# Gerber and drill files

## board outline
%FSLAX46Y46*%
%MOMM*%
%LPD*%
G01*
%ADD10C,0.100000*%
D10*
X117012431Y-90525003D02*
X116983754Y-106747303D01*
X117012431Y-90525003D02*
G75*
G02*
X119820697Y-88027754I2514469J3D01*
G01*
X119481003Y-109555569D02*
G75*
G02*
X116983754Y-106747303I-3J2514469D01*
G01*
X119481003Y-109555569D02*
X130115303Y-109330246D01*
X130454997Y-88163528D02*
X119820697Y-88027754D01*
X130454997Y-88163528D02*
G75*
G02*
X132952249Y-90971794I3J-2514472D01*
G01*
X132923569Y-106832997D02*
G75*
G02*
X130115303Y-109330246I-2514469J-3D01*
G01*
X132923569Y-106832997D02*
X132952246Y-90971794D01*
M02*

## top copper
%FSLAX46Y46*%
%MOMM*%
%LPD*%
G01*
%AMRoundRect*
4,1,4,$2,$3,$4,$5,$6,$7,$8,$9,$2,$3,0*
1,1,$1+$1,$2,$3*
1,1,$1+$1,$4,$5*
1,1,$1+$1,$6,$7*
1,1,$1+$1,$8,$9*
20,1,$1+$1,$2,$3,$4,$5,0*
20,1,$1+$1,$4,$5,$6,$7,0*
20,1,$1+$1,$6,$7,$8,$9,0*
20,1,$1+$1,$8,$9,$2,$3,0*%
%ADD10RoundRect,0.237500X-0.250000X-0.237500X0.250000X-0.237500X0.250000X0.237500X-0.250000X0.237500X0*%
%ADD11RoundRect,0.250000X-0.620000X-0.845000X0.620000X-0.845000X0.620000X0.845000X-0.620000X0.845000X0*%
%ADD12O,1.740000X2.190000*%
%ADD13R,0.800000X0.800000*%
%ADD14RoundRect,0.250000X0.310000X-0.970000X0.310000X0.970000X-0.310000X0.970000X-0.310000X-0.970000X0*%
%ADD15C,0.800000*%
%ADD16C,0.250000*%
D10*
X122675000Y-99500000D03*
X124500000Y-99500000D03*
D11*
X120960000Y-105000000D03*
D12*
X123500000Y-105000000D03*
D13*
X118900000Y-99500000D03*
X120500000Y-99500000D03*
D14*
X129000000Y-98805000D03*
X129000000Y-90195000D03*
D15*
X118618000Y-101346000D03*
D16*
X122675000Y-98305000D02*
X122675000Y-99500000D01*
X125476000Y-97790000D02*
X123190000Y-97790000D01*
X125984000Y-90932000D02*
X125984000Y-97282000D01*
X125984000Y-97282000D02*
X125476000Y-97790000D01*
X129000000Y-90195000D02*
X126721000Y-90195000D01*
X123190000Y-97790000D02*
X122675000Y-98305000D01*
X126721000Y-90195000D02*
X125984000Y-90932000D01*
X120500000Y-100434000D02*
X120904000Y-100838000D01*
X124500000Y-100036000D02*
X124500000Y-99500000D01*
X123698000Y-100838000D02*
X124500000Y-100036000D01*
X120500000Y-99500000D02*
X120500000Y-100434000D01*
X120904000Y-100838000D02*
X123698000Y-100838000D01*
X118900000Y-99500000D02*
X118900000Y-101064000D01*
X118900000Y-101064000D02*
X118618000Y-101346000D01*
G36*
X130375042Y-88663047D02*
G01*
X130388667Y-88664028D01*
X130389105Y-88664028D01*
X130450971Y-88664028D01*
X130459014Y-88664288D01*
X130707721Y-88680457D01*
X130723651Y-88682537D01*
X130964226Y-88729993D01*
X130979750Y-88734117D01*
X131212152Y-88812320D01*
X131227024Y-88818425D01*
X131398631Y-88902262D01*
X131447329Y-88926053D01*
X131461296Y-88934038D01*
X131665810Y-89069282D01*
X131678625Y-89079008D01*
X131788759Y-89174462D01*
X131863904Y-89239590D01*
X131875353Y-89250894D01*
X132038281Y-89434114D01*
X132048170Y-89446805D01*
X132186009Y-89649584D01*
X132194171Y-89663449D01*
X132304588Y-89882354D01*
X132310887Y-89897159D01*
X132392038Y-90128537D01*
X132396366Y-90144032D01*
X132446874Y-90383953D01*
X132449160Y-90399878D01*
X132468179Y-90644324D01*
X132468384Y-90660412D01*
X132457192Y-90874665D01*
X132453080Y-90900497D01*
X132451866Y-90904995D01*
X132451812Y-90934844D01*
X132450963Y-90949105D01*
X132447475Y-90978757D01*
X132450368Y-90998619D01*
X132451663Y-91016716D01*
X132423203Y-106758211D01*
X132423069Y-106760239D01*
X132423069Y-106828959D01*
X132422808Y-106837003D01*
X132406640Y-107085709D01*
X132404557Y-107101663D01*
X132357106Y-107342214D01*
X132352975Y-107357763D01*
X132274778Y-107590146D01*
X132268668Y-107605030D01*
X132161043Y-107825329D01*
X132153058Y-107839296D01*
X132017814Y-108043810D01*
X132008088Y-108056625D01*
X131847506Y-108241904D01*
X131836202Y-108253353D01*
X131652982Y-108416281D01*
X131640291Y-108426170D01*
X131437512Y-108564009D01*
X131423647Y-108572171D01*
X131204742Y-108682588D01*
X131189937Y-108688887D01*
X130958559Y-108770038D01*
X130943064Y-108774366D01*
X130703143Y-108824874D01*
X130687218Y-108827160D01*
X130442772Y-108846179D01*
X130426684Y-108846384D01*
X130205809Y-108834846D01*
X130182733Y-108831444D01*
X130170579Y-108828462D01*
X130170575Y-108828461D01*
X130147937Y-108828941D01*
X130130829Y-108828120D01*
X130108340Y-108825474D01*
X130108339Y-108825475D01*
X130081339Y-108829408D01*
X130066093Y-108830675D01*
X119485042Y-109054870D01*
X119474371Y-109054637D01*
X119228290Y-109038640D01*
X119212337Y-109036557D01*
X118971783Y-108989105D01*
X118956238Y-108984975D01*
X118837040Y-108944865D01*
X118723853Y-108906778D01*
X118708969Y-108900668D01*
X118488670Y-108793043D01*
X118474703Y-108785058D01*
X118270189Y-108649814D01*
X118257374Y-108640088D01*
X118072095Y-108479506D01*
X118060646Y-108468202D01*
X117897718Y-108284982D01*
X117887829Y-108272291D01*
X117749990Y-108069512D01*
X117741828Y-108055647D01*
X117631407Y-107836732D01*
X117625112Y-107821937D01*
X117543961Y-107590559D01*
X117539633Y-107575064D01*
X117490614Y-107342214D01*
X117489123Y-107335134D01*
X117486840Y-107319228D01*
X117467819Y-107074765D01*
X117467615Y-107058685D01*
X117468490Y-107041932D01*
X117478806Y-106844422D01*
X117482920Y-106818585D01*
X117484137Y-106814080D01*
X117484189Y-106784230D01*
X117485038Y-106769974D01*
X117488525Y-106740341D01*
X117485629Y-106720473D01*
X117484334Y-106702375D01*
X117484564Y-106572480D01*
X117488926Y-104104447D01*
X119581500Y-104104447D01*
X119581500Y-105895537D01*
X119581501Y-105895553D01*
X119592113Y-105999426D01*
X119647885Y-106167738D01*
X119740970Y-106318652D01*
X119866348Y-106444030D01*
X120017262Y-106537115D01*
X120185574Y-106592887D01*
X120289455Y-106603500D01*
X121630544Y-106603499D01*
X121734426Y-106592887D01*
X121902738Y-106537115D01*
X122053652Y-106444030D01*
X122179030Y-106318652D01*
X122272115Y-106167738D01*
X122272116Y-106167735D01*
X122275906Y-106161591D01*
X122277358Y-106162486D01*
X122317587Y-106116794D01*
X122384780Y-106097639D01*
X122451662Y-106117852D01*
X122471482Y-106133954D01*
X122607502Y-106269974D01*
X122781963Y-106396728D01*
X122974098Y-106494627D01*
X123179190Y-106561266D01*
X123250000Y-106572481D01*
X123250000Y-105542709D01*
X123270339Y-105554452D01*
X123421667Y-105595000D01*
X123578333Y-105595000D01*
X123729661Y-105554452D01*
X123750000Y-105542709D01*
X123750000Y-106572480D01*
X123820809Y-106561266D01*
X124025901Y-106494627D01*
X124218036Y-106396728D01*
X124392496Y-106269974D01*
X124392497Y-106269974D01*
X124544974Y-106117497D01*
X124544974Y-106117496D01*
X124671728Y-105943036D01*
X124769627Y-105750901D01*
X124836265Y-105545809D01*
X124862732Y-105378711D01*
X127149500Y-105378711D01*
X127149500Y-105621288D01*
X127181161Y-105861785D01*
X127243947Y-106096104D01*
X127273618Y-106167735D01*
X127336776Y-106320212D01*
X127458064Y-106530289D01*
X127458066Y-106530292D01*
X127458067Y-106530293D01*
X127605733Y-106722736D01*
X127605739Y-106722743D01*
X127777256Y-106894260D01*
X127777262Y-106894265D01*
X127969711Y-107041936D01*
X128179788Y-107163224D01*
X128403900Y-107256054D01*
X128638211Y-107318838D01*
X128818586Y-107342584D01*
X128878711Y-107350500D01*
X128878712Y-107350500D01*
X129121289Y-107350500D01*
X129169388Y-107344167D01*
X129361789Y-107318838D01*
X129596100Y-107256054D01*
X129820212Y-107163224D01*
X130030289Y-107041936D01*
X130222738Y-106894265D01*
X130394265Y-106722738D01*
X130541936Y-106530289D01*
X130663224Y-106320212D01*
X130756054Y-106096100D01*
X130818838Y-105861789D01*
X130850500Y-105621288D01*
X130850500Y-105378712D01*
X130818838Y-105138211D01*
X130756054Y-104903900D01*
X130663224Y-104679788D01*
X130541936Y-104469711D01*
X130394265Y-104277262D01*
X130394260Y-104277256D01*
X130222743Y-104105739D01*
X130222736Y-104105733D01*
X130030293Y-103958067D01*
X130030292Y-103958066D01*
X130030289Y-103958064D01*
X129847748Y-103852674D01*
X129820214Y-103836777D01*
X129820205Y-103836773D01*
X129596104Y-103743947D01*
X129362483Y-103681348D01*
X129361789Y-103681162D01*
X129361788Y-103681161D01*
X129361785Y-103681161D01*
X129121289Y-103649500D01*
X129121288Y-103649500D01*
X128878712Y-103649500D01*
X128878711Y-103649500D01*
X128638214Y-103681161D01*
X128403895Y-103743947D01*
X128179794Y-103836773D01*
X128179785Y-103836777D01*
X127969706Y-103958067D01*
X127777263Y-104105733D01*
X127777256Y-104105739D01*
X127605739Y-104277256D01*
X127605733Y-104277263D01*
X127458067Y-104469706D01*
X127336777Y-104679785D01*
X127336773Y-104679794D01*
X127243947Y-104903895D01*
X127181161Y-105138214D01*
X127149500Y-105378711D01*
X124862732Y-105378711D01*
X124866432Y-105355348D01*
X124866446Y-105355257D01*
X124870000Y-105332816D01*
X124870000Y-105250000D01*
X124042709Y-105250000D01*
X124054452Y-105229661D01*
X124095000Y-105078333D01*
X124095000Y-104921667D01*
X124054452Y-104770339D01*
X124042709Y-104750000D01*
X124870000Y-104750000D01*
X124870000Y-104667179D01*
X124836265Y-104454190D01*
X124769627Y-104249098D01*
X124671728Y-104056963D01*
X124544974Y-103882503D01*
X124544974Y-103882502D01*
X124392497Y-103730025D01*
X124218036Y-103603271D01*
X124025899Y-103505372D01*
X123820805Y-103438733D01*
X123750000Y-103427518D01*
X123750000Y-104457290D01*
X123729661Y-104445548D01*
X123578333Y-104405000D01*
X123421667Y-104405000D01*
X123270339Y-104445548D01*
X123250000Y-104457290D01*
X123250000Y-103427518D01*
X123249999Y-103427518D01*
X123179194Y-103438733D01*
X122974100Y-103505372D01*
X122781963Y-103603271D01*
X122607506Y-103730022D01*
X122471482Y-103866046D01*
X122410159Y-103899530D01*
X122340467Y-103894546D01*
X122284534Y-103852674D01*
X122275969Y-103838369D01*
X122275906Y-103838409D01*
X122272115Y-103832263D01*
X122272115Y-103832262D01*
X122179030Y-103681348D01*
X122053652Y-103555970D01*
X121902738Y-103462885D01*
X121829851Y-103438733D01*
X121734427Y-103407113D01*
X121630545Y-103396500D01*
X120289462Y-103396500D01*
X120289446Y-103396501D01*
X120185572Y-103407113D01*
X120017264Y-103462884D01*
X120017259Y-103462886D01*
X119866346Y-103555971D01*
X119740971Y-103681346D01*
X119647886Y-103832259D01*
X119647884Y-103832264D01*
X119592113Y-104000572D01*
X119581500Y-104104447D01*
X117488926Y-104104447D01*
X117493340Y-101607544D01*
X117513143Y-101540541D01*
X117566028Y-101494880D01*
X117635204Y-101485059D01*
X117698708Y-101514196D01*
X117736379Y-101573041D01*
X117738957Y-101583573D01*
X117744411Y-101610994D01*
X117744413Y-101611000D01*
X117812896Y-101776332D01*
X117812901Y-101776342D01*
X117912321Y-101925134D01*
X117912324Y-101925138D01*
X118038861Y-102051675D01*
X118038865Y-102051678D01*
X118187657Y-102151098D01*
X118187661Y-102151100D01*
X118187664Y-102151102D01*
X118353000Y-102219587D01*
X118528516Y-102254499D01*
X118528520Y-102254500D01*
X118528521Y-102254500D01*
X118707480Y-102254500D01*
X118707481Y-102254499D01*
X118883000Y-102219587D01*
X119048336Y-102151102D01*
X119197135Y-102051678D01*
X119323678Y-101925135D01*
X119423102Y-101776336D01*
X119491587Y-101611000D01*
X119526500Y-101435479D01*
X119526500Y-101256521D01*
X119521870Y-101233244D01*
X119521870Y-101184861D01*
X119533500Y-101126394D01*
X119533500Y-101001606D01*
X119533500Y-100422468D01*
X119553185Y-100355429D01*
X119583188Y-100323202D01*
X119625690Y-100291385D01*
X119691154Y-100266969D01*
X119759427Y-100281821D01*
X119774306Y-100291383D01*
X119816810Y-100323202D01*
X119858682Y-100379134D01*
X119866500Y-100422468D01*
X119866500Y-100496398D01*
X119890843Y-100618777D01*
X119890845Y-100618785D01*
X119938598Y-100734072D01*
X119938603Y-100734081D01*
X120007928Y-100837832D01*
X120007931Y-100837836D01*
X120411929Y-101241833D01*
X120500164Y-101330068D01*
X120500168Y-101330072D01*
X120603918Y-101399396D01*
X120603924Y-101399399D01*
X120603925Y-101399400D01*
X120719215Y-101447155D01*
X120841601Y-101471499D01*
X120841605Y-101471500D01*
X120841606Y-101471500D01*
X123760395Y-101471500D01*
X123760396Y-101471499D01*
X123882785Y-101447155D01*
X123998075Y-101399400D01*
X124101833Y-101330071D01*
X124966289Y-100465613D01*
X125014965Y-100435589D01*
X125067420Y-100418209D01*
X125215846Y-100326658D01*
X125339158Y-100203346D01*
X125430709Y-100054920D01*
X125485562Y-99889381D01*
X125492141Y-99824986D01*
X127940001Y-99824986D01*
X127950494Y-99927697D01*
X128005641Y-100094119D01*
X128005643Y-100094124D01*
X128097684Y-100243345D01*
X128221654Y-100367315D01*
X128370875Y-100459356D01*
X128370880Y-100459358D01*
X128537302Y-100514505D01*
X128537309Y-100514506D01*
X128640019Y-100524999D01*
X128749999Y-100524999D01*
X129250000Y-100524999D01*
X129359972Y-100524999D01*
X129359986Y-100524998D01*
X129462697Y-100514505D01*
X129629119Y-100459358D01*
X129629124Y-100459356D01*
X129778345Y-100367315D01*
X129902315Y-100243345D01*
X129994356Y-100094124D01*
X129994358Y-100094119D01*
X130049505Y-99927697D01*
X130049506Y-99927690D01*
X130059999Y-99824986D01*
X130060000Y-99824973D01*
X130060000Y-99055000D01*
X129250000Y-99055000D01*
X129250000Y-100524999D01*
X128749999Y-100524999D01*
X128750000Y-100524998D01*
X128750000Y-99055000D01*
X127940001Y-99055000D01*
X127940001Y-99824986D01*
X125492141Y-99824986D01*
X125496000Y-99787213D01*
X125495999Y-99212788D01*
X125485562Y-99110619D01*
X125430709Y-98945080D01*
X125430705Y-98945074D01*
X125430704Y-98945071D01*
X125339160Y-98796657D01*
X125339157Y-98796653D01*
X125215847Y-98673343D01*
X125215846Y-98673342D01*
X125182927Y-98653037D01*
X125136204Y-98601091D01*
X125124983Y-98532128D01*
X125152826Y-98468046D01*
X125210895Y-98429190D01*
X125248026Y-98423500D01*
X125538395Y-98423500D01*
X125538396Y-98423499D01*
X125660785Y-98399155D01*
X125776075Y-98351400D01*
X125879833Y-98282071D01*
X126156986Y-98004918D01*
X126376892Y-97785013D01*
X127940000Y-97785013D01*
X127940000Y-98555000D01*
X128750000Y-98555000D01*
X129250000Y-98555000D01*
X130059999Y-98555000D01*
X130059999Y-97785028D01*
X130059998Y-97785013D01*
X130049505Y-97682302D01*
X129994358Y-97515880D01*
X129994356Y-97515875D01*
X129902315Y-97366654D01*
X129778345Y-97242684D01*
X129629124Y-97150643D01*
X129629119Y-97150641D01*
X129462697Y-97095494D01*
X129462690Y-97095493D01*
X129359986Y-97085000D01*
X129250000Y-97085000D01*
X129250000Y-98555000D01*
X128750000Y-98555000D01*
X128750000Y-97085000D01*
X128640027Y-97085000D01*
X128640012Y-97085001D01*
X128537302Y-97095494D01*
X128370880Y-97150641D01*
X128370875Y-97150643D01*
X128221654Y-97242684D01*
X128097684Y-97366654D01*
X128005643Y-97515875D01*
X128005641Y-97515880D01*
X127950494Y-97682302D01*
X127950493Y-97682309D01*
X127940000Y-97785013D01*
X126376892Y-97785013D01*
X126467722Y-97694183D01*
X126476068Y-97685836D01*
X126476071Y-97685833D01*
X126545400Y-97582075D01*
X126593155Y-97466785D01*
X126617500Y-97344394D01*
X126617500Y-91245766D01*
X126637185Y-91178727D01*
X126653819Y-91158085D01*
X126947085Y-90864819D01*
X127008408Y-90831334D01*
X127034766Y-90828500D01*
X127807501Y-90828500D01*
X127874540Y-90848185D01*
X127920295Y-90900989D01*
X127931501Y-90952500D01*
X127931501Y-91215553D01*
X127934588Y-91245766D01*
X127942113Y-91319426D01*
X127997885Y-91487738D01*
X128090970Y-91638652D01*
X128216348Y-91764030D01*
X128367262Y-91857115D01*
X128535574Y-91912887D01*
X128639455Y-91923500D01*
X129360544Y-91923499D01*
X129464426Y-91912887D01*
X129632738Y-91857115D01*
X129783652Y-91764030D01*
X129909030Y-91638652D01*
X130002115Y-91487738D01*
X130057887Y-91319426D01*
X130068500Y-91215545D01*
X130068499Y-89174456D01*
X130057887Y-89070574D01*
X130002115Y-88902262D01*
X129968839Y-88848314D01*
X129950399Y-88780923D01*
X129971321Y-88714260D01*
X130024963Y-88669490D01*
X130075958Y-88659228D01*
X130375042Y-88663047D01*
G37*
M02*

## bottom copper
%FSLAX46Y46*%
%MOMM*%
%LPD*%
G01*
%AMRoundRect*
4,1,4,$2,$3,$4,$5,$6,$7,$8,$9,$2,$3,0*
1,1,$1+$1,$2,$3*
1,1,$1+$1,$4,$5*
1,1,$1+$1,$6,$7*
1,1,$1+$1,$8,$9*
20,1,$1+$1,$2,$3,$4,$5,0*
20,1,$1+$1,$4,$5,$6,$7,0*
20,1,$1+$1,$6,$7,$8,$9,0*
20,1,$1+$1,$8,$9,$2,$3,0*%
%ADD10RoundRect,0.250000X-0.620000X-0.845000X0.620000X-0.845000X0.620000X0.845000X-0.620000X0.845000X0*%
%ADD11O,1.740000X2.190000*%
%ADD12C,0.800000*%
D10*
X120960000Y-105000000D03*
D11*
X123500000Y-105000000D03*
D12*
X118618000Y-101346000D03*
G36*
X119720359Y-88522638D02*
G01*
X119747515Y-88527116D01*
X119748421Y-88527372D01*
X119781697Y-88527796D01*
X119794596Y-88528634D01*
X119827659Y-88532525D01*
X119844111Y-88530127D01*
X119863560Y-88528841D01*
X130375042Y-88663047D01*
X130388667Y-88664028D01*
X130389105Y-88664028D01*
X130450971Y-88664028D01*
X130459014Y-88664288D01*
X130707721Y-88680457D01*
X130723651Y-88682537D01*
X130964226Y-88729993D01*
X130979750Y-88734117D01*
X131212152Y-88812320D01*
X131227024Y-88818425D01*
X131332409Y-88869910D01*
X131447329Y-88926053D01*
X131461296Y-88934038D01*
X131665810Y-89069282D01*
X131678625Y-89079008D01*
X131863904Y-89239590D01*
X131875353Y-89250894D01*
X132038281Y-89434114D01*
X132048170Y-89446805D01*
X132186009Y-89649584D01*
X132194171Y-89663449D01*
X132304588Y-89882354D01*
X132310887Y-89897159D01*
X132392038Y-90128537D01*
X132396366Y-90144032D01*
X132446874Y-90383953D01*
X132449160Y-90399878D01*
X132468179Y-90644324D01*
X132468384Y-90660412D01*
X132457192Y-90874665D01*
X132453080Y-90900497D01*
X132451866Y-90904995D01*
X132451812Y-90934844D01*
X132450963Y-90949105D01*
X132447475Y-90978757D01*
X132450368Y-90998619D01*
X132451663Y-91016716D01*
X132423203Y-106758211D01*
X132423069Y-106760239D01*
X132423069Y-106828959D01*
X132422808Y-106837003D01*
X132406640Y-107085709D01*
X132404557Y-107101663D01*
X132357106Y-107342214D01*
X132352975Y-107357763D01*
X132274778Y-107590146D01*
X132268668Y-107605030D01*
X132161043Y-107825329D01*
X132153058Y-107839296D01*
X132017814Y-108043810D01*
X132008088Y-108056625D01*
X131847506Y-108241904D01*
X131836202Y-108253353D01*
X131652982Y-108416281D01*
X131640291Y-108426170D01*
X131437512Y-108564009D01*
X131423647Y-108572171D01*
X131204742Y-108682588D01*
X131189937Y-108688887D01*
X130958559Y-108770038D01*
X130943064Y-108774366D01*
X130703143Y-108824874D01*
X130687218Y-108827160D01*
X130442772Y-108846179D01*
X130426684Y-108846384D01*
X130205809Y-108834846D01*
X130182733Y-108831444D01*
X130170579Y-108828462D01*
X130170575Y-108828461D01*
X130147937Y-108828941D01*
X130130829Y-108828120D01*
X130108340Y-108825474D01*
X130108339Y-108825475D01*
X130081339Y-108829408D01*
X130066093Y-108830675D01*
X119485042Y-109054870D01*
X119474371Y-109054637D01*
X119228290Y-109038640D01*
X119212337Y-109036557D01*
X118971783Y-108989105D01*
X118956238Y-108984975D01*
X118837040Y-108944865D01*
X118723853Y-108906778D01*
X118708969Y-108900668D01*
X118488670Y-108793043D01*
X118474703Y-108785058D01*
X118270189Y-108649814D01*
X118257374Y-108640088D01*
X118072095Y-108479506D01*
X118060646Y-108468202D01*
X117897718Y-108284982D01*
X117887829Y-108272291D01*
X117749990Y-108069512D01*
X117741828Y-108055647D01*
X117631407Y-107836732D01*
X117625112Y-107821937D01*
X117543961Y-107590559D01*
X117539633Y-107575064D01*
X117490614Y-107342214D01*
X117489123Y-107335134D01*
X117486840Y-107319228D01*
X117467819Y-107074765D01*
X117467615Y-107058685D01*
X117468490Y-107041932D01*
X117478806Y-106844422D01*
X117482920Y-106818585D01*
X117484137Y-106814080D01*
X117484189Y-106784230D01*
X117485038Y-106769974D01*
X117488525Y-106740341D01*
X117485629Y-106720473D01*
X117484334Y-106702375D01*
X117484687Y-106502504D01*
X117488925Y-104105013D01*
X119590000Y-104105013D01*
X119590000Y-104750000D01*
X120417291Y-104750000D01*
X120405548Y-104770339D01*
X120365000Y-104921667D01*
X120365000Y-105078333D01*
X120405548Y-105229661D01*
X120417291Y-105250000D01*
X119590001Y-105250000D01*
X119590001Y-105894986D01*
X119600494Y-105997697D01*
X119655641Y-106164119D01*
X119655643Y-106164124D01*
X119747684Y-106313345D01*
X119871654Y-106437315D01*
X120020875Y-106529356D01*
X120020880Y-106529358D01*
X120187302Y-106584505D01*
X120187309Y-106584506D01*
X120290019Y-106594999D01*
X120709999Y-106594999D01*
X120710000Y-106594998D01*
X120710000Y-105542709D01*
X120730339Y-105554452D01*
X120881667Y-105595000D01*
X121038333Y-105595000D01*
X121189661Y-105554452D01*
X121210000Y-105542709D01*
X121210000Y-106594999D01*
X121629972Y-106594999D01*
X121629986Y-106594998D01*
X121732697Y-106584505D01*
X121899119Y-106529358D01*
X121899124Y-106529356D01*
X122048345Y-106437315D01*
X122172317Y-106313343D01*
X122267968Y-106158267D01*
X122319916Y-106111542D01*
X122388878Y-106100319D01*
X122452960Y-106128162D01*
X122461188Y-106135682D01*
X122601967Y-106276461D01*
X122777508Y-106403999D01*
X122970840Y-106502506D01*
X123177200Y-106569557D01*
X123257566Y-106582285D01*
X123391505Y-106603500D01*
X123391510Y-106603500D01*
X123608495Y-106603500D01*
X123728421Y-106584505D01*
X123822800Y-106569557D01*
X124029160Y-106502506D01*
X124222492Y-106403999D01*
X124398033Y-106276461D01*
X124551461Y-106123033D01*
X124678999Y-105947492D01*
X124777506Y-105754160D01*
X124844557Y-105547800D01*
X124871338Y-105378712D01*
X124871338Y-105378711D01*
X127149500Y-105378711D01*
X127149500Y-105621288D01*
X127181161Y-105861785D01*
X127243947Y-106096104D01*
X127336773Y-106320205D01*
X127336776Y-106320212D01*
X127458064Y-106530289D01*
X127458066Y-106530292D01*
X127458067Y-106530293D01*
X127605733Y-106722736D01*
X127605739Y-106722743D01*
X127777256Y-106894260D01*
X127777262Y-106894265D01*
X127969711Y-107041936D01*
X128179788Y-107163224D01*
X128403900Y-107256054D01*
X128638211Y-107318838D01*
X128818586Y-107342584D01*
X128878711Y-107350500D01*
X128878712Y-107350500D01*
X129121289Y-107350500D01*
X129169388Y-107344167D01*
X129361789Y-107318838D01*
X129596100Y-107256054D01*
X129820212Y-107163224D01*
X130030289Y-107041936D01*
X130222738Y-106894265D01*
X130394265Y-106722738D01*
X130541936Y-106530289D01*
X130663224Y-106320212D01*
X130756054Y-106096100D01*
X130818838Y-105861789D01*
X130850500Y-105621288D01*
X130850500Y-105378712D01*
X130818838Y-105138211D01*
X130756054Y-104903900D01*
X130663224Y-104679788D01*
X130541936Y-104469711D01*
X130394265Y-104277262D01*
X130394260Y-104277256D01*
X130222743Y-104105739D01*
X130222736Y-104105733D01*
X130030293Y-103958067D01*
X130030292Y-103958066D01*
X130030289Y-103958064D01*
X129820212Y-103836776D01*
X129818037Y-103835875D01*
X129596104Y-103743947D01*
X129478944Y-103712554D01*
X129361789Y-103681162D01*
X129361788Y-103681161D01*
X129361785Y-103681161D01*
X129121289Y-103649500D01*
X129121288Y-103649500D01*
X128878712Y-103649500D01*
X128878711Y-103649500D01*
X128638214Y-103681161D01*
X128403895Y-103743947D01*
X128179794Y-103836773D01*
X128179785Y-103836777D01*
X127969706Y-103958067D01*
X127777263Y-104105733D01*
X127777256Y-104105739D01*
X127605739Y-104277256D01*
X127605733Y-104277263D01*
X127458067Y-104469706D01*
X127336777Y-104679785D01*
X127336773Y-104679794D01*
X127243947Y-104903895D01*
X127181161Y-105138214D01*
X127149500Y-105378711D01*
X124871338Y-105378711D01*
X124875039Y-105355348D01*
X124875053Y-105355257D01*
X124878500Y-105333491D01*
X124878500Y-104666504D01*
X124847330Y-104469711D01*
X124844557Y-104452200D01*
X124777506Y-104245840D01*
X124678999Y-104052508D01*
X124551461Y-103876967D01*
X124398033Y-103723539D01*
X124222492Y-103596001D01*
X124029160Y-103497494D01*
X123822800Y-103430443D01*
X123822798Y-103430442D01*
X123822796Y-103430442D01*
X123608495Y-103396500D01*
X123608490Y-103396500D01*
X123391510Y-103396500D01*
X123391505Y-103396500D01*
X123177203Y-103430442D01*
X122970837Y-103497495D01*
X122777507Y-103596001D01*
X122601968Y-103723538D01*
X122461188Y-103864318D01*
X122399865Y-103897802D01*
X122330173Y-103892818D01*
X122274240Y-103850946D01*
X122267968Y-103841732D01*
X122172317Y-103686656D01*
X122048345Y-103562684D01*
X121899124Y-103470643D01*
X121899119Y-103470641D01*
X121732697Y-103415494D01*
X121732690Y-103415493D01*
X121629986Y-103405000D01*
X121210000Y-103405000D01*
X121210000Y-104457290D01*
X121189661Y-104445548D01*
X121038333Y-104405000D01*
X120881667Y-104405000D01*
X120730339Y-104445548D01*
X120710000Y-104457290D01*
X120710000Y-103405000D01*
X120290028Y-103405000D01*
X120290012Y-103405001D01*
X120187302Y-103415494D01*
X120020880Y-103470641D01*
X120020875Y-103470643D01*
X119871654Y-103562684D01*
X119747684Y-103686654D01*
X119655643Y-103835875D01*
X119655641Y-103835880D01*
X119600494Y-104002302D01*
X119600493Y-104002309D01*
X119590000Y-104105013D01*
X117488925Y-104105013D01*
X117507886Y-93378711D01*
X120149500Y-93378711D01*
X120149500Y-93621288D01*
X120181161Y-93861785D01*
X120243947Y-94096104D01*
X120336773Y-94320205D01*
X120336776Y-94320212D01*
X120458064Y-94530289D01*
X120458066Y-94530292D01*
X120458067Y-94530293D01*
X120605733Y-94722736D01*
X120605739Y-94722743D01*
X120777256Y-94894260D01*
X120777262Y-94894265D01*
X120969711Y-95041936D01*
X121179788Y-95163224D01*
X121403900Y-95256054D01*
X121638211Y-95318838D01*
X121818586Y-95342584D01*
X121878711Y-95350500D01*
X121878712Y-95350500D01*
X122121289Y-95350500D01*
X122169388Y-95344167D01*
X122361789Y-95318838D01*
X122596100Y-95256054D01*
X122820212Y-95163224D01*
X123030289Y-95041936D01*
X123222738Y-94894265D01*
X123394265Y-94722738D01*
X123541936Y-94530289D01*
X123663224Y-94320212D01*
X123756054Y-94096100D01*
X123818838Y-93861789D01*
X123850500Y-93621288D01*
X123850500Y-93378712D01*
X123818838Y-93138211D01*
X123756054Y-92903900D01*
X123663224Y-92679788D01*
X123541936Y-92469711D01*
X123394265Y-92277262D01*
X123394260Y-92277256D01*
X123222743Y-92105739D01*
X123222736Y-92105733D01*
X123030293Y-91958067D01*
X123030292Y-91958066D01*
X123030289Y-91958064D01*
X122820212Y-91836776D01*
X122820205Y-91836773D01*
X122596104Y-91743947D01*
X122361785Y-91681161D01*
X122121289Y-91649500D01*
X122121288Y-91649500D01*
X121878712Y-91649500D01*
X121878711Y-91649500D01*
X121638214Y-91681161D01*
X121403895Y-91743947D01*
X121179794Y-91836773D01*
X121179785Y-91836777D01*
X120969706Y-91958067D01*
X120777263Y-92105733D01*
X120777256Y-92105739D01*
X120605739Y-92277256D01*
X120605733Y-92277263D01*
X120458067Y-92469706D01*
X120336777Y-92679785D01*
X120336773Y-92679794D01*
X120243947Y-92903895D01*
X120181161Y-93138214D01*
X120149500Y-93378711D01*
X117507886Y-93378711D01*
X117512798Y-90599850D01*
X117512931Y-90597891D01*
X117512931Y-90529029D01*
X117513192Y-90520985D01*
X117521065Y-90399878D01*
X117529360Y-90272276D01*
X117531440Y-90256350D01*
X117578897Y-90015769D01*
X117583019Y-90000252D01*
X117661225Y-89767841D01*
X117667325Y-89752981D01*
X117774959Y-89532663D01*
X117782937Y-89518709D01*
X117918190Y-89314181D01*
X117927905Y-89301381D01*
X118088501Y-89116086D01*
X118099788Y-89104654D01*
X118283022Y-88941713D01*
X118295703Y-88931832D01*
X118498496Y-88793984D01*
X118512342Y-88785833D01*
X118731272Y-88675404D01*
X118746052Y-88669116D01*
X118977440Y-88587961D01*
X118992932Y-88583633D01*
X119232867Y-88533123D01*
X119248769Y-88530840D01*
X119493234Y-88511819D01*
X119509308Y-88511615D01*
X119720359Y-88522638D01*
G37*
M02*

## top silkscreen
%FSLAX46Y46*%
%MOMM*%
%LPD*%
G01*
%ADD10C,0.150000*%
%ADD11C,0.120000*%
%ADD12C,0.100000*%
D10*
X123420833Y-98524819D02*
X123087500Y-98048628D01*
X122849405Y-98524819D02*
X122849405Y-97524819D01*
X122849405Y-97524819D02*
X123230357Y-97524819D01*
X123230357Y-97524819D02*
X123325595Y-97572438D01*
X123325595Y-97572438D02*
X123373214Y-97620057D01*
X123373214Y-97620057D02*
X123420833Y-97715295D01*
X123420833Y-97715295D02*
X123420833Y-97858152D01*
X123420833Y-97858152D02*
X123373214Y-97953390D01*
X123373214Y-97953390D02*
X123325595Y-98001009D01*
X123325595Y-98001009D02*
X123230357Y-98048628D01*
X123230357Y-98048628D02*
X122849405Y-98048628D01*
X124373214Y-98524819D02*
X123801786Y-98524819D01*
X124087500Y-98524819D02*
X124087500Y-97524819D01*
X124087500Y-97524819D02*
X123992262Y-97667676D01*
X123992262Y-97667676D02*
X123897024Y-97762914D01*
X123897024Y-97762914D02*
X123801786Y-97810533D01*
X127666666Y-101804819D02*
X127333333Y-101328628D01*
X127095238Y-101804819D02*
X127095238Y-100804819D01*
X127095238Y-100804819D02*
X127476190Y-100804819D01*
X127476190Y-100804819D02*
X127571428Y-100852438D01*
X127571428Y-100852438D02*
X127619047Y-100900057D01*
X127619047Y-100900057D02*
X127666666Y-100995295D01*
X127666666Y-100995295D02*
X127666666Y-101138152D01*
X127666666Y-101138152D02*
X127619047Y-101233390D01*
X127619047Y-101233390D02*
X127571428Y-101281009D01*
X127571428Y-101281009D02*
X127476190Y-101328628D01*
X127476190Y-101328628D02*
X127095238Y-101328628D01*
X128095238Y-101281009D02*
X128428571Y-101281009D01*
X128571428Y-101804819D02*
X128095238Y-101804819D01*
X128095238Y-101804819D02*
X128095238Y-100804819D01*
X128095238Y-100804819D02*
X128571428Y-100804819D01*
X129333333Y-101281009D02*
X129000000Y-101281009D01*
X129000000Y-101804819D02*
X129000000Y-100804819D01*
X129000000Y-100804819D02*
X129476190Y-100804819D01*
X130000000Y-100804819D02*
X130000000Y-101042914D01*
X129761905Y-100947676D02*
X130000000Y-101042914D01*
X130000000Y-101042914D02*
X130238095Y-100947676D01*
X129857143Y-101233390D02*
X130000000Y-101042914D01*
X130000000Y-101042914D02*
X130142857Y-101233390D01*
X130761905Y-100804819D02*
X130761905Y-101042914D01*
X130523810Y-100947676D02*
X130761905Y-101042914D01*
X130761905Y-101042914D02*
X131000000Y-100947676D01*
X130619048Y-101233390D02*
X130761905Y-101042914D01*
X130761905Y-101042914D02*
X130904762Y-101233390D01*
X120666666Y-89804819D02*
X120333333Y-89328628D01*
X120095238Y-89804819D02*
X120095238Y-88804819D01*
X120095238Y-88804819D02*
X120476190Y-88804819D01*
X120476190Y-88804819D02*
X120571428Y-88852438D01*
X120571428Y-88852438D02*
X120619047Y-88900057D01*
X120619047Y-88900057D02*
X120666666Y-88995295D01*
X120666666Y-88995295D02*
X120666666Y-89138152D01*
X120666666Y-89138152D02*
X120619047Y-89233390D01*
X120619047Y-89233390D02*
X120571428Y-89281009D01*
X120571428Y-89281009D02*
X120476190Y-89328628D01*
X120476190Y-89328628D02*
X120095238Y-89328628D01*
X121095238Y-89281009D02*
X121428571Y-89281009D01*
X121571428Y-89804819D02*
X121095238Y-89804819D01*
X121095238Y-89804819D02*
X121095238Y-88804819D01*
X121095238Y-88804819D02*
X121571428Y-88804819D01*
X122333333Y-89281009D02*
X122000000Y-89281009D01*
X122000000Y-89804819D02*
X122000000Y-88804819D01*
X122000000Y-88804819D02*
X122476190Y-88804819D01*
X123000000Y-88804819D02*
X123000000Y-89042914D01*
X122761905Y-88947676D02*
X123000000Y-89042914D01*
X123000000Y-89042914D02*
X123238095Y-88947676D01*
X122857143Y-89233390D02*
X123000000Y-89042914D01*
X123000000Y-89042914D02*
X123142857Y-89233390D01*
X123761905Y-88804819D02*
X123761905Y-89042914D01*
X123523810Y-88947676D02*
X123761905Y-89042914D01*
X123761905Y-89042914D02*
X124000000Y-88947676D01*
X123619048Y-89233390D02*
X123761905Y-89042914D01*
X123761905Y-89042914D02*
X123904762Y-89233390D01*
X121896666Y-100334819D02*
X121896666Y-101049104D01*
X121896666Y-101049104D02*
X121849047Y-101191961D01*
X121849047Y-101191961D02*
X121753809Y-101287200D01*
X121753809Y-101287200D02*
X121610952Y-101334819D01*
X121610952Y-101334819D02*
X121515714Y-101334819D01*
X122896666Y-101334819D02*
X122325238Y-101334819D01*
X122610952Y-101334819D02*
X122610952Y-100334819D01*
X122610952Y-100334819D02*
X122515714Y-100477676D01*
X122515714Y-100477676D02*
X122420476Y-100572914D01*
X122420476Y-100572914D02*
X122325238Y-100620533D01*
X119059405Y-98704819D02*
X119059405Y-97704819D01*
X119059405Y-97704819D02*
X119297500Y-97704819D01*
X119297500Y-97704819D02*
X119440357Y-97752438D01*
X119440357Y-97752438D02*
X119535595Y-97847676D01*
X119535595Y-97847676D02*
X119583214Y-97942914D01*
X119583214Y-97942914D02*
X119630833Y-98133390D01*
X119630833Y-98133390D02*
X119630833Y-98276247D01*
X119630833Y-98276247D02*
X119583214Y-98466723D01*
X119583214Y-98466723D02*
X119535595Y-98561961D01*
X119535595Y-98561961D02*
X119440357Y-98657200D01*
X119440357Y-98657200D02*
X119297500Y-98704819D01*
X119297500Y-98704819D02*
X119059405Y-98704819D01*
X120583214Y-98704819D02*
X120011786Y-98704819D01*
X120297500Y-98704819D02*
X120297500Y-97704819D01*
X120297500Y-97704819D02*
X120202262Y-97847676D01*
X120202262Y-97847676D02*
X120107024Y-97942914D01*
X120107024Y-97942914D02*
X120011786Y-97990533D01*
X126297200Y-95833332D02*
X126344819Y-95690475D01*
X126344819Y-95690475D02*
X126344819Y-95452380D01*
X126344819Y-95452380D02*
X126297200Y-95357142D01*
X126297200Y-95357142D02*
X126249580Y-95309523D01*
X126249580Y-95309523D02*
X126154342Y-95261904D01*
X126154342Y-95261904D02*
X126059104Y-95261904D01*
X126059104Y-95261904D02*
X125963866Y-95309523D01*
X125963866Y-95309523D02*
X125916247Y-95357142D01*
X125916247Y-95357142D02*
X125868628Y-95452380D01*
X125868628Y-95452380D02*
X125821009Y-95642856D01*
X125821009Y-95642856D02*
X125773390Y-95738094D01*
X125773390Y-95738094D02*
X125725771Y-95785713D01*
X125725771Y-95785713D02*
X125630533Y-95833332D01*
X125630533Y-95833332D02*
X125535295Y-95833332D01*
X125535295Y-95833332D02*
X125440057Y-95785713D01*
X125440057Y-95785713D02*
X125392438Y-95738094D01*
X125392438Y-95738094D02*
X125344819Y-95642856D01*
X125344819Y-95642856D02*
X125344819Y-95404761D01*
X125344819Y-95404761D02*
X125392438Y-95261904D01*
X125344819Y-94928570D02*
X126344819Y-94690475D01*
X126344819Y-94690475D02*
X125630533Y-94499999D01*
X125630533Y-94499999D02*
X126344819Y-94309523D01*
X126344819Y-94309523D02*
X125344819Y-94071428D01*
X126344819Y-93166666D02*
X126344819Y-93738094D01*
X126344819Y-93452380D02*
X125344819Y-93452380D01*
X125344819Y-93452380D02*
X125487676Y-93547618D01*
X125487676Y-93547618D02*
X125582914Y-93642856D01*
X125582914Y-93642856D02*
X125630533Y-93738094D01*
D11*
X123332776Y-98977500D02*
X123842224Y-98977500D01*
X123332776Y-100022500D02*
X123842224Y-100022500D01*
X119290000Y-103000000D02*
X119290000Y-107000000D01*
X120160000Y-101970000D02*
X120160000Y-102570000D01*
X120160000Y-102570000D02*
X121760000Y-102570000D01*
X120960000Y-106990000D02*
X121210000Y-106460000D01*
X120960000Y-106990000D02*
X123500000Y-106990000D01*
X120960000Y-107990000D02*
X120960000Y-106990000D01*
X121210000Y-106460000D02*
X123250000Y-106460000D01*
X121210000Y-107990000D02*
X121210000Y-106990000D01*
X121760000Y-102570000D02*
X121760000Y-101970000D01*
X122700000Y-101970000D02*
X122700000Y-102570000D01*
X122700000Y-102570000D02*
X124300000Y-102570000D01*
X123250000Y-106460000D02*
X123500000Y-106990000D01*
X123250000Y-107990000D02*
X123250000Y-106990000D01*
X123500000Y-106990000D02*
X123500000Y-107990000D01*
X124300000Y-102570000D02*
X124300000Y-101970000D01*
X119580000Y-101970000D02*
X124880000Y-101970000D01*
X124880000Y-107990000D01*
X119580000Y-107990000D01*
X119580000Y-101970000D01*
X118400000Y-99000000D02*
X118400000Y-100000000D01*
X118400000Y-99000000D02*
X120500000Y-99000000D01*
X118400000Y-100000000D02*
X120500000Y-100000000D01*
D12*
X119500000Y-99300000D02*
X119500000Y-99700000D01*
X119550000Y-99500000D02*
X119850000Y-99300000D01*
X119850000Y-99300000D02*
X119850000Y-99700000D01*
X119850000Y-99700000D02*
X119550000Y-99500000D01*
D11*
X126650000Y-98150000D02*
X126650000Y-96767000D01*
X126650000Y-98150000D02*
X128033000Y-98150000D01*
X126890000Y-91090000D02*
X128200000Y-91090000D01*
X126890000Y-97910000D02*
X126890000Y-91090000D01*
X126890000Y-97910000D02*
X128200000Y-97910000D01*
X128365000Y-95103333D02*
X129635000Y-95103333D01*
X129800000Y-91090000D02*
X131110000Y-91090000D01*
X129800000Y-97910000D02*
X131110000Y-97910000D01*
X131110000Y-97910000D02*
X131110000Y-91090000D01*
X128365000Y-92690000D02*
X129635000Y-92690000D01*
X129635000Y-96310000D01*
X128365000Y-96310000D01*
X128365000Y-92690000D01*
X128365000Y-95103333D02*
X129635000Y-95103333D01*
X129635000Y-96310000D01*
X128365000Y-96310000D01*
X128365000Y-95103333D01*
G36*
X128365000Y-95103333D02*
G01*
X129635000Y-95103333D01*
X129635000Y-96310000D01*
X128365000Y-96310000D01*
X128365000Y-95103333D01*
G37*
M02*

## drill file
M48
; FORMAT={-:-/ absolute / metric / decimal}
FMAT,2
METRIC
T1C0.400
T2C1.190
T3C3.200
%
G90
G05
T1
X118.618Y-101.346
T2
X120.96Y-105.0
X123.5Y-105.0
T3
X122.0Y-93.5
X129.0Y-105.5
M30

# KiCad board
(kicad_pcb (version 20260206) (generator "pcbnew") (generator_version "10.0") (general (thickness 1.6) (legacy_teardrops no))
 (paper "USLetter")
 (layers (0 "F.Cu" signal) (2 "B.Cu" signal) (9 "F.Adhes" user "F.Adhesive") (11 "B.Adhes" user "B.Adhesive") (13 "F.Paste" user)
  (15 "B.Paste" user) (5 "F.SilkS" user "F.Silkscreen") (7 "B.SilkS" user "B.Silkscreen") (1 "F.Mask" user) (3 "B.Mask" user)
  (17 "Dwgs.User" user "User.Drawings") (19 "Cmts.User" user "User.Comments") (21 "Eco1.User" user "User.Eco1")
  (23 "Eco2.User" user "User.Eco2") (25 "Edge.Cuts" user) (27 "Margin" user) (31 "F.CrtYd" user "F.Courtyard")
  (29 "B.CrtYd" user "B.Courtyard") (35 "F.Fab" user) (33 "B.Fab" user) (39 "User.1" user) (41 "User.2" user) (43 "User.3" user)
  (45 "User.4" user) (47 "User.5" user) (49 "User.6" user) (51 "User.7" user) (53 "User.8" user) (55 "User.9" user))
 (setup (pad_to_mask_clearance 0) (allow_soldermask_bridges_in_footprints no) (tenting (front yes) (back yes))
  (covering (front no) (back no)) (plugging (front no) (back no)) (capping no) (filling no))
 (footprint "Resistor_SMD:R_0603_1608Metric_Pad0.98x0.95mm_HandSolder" (layer "F.Cu") (at 123.5875 99.5)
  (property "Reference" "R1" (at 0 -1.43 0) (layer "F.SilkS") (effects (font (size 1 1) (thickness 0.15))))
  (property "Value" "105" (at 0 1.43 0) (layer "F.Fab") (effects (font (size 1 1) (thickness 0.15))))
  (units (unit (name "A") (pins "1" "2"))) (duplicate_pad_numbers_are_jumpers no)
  (fp_line (start -0.254724 -0.5225) (end 0.254724 -0.5225) (stroke (width 0.12) (type solid)) (layer "F.SilkS"))
  (fp_line (start -0.254724 0.5225) (end 0.254724 0.5225) (stroke (width 0.12) (type solid)) (layer "F.SilkS"))
  (pad "1" smd roundrect (at -0.9125 0) (size 0.975 0.95) (layers "F.Cu" "F.Mask" "F.Paste") (roundrect_rratio 0.25) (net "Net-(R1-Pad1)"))
  (pad "2" smd roundrect (at 0.9125 0) (size 0.975 0.95) (layers "F.Cu" "F.Mask" "F.Paste") (roundrect_rratio 0.25) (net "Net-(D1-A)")))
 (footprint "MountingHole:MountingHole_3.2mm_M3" (layer "F.Cu") (at 129 105.5)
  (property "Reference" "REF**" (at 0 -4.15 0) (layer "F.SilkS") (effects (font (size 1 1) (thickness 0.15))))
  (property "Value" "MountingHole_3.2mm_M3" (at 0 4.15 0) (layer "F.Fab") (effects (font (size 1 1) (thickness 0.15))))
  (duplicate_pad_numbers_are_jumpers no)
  (pad "" np_thru_hole circle (at 0 0) (size 3.2 3.2) (drill 3.2) (layers "*.Cu" "*.Mask")))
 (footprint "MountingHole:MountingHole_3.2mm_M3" (layer "F.Cu") (at 122 93.5)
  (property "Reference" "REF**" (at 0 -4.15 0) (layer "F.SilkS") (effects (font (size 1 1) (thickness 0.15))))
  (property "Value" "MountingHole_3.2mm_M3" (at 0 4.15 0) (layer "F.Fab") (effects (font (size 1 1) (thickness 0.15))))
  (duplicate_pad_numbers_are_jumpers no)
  (pad "" np_thru_hole circle (at 0 0) (size 3.2 3.2) (drill 3.2) (layers "*.Cu" "*.Mask")))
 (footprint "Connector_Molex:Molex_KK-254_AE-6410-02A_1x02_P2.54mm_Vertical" (layer "F.Cu") (at 120.96 105)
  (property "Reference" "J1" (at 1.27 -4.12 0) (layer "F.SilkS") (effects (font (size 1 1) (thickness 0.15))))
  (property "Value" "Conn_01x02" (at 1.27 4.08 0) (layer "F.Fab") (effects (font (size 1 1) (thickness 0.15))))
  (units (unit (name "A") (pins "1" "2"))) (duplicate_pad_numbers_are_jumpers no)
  (fp_line (start -1.67 -2) (end -1.67 2) (stroke (width 0.12) (type solid)) (layer "F.SilkS"))
  (fp_line (start -0.8 -3.03) (end -0.8 -2.43) (stroke (width 0.12) (type solid)) (layer "F.SilkS"))
  (fp_line (start -0.8 -2.43) (end 0.8 -2.43) (stroke (width 0.12) (type solid)) (layer "F.SilkS"))
  (fp_line (start 0 1.99) (end 0.25 1.46) (stroke (width 0.12) (type solid)) (layer "F.SilkS"))
  (fp_line (start 0 1.99) (end 2.54 1.99) (stroke (width 0.12) (type solid)) (layer "F.SilkS"))
  (fp_line (start 0 2.99) (end 0 1.99) (stroke (width 0.12) (type solid)) (layer "F.SilkS"))
  (fp_line (start 0.25 1.46) (end 2.29 1.46) (stroke (width 0.12) (type solid)) (layer "F.SilkS"))
  (fp_line (start 0.25 2.99) (end 0.25 1.99) (stroke (width 0.12) (type solid)) (layer "F.SilkS"))
  (fp_line (start 0.8 -2.43) (end 0.8 -3.03) (stroke (width 0.12) (type solid)) (layer "F.SilkS"))
  (fp_line (start 1.74 -3.03) (end 1.74 -2.43) (stroke (width 0.12) (type solid)) (layer "F.SilkS"))
  (fp_line (start 1.74 -2.43) (end 3.34 -2.43) (stroke (width 0.12) (type solid)) (layer "F.SilkS"))
  (fp_line (start 2.29 1.46) (end 2.54 1.99) (stroke (width 0.12) (type solid)) (layer "F.SilkS"))
  (fp_line (start 2.29 2.99) (end 2.29 1.99) (stroke (width 0.12) (type solid)) (layer "F.SilkS"))
  (fp_line (start 2.54 1.99) (end 2.54 2.99) (stroke (width 0.12) (type solid)) (layer "F.SilkS"))
  (fp_line (start 3.34 -2.43) (end 3.34 -3.03) (stroke (width 0.12) (type solid)) (layer "F.SilkS"))
  (fp_rect (start -1.38 -3.03) (end 3.92 2.99) (stroke (width 0.12) (type solid)) (fill no) (layer "F.SilkS"))
  (pad "1" thru_hole roundrect (at 0 0) (size 1.74 2.19) (drill 1.19) (layers "*.Cu" "*.Mask") (remove_unused_layers no)
   (roundrect_rratio 0.143678) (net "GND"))
  (pad "2" thru_hole oval (at 2.54 0) (size 1.74 2.19) (drill 1.19) (layers "*.Cu" "*.Mask") (remove_unused_layers no) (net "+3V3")))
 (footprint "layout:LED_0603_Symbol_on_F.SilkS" (layer "F.Cu") (at 119.7 99.5)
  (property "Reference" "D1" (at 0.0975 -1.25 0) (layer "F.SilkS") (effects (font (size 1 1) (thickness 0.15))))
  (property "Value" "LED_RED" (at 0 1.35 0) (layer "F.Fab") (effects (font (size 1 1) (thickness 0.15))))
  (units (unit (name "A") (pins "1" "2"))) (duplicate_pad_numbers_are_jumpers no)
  (fp_line (start -1.3 -0.5) (end -1.3 0.5) (stroke (width 0.12) (type solid)) (layer "F.SilkS"))
  (fp_line (start -1.3 -0.5) (end 0.8 -0.5) (stroke (width 0.12) (type solid)) (layer "F.SilkS"))
  (fp_line (start -1.3 0.5) (end 0.8 0.5) (stroke (width 0.12) (type solid)) (layer "F.SilkS"))
  (fp_line (start -0.2 -0.2) (end -0.2 0.2) (stroke (width 0.1) (type solid)) (layer "F.SilkS"))
  (fp_line (start -0.15 0) (end 0.15 -0.2) (stroke (width 0.1) (type solid)) (layer "F.SilkS"))
  (fp_line (start 0.15 -0.2) (end 0.15 0.2) (stroke (width 0.1) (type solid)) (layer "F.SilkS"))
  (fp_line (start 0.15 0.2) (end -0.15 0) (stroke (width 0.1) (type solid)) (layer "F.SilkS"))
  (pad "1" smd rect (at -0.8 0 180) (size 0.8 0.8) (layers "F.Cu" "F.Mask" "F.Paste") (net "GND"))
  (pad "2" smd rect (at 0.8 0 180) (size 0.8 0.8) (layers "F.Cu" "F.Mask" "F.Paste") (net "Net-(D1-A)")))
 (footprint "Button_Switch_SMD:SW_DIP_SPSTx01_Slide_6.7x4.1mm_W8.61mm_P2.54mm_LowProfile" (layer "F.Cu") (at 129 94.5 90)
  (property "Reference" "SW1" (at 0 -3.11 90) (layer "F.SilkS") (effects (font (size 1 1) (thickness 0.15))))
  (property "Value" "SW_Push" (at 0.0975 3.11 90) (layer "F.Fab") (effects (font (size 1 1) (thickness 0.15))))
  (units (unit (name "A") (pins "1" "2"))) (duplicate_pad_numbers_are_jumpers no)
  (fp_line (start -3.65 -2.35) (end -2.267 -2.35) (stroke (width 0.12) (type solid)) (layer "F.SilkS"))
  (fp_line (start -3.65 -2.35) (end -3.65 -0.967) (stroke (width 0.12) (type solid)) (layer "F.SilkS"))
  (fp_line (start 3.41 -2.11) (end 3.41 -0.8) (stroke (width 0.12) (type solid)) (layer "F.SilkS"))
  (fp_line (start -3.41 -2.11) (end 3.41 -2.11) (stroke (width 0.12) (type solid)) (layer "F.SilkS"))
  (fp_line (start -3.41 -2.11) (end -3.41 -0.8) (stroke (width 0.12) (type solid)) (layer "F.SilkS"))
  (fp_line (start -0.603333 -0.635) (end -0.603333 0.635) (stroke (width 0.12) (type solid)) (layer "F.SilkS"))
  (fp_line (start 3.41 0.8) (end 3.41 2.11) (stroke (width 0.12) (type solid)) (layer "F.SilkS"))
  (fp_line (start -3.41 0.8) (end -3.41 2.11) (stroke (width 0.12) (type solid)) (layer "F.SilkS"))
  (fp_line (start -3.41 2.11) (end 3.41 2.11) (stroke (width 0.12) (type solid)) (layer "F.SilkS"))
  (fp_rect (start -1.81 -0.635) (end 1.81 0.635) (stroke (width 0.12) (type solid)) (fill no) (layer "F.SilkS"))
  (fp_rect (start -1.81 -0.635) (end -0.603333 0.635) (stroke (width 0.12) (type solid)) (fill yes) (layer "F.SilkS"))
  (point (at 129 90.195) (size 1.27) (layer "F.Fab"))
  (pad "1" smd roundrect (at -4.305 0 90) (size 2.44 1.12) (layers "F.Cu" "F.Mask" "F.Paste") (roundrect_rratio 0.223214) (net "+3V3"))
  (pad "2" smd roundrect (at 4.305 0 90) (size 2.44 1.12) (layers "F.Cu" "F.Mask" "F.Paste") (roundrect_rratio 0.223214)
   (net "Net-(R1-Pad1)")))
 (gr_line (start 117.012431 90.525003) (end 116.983754 106.747303) (stroke (width 0.1) (type default)) (layer "Edge.Cuts"))
 (gr_arc (start 117.012431 90.525003) (mid 117.856 88.646) (end 119.820697 88.027754) (stroke (width 0.1) (type default))
  (layer "Edge.Cuts"))
 (gr_arc (start 119.481003 109.555569) (mid 117.602 108.712) (end 116.983754 106.747303) (stroke (width 0.1) (type default))
  (layer "Edge.Cuts"))
 (gr_line (start 119.481003 109.555569) (end 130.115303 109.330246) (stroke (width 0.1) (type default)) (layer "Edge.Cuts"))
 (gr_line (start 130.454997 88.163528) (end 119.820697 88.027754) (stroke (width 0.1) (type default)) (layer "Edge.Cuts"))
 (gr_arc (start 130.454997 88.163528) (mid 132.334 89.007097) (end 132.952246 90.971794) (stroke (width 0.1) (type default))
  (layer "Edge.Cuts"))
 (gr_arc (start 132.923569 106.832997) (mid 132.08 108.712) (end 130.115303 109.330246) (stroke (width 0.1) (type default))
  (layer "Edge.Cuts"))
 (gr_line (start 132.923569 106.832997) (end 132.952246 90.971794) (stroke (width 0.1) (type default)) (layer "Edge.Cuts"))
 (segment (start 122.675 98.305) (end 122.675 99.5) (width 0.25) (layer "F.Cu") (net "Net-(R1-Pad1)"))
 (segment (start 125.476 97.79) (end 123.19 97.79) (width 0.25) (layer "F.Cu") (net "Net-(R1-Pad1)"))
 (segment (start 125.984 90.932) (end 125.984 97.282) (width 0.25) (layer "F.Cu") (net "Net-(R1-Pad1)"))
 (segment (start 125.984 97.282) (end 125.476 97.79) (width 0.25) (layer "F.Cu") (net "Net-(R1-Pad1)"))
 (segment (start 129 90.195) (end 126.721 90.195) (width 0.25) (layer "F.Cu") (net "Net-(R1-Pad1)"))
 (segment (start 123.19 97.79) (end 122.675 98.305) (width 0.25) (layer "F.Cu") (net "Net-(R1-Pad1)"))
 (segment (start 126.721 90.195) (end 125.984 90.932) (width 0.25) (layer "F.Cu") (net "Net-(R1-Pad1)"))
 (segment (start 120.5 100.434) (end 120.904 100.838) (width 0.25) (layer "F.Cu") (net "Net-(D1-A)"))
 (segment (start 124.5 100.036) (end 124.5 99.5) (width 0.25) (layer "F.Cu") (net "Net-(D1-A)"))
 (segment (start 123.698 100.838) (end 124.5 100.036) (width 0.25) (layer "F.Cu") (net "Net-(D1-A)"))
 (segment (start 120.5 99.5) (end 120.5 100.434) (width 0.25) (layer "F.Cu") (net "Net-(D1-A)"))
 (segment (start 120.904 100.838) (end 123.698 100.838) (width 0.25) (layer "F.Cu") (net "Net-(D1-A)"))
 (segment (start 118.9 99.5) (end 118.9 101.064) (width 0.25) (layer "F.Cu") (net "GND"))
 (segment (start 118.9 101.064) (end 118.618 101.346) (width 0.25) (layer "F.Cu") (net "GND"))
 (via (at 118.618 101.346) (size 0.8) (drill 0.4) (layers "F.Cu" "B.Cu") (free yes) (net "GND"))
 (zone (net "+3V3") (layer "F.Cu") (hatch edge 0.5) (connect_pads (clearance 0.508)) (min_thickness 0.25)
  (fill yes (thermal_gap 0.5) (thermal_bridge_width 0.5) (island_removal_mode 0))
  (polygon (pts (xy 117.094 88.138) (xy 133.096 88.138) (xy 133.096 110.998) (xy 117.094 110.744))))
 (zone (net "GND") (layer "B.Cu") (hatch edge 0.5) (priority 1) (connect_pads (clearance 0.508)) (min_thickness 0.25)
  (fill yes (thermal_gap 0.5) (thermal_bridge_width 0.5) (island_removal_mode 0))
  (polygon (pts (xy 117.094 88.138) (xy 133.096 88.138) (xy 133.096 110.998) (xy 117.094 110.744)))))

